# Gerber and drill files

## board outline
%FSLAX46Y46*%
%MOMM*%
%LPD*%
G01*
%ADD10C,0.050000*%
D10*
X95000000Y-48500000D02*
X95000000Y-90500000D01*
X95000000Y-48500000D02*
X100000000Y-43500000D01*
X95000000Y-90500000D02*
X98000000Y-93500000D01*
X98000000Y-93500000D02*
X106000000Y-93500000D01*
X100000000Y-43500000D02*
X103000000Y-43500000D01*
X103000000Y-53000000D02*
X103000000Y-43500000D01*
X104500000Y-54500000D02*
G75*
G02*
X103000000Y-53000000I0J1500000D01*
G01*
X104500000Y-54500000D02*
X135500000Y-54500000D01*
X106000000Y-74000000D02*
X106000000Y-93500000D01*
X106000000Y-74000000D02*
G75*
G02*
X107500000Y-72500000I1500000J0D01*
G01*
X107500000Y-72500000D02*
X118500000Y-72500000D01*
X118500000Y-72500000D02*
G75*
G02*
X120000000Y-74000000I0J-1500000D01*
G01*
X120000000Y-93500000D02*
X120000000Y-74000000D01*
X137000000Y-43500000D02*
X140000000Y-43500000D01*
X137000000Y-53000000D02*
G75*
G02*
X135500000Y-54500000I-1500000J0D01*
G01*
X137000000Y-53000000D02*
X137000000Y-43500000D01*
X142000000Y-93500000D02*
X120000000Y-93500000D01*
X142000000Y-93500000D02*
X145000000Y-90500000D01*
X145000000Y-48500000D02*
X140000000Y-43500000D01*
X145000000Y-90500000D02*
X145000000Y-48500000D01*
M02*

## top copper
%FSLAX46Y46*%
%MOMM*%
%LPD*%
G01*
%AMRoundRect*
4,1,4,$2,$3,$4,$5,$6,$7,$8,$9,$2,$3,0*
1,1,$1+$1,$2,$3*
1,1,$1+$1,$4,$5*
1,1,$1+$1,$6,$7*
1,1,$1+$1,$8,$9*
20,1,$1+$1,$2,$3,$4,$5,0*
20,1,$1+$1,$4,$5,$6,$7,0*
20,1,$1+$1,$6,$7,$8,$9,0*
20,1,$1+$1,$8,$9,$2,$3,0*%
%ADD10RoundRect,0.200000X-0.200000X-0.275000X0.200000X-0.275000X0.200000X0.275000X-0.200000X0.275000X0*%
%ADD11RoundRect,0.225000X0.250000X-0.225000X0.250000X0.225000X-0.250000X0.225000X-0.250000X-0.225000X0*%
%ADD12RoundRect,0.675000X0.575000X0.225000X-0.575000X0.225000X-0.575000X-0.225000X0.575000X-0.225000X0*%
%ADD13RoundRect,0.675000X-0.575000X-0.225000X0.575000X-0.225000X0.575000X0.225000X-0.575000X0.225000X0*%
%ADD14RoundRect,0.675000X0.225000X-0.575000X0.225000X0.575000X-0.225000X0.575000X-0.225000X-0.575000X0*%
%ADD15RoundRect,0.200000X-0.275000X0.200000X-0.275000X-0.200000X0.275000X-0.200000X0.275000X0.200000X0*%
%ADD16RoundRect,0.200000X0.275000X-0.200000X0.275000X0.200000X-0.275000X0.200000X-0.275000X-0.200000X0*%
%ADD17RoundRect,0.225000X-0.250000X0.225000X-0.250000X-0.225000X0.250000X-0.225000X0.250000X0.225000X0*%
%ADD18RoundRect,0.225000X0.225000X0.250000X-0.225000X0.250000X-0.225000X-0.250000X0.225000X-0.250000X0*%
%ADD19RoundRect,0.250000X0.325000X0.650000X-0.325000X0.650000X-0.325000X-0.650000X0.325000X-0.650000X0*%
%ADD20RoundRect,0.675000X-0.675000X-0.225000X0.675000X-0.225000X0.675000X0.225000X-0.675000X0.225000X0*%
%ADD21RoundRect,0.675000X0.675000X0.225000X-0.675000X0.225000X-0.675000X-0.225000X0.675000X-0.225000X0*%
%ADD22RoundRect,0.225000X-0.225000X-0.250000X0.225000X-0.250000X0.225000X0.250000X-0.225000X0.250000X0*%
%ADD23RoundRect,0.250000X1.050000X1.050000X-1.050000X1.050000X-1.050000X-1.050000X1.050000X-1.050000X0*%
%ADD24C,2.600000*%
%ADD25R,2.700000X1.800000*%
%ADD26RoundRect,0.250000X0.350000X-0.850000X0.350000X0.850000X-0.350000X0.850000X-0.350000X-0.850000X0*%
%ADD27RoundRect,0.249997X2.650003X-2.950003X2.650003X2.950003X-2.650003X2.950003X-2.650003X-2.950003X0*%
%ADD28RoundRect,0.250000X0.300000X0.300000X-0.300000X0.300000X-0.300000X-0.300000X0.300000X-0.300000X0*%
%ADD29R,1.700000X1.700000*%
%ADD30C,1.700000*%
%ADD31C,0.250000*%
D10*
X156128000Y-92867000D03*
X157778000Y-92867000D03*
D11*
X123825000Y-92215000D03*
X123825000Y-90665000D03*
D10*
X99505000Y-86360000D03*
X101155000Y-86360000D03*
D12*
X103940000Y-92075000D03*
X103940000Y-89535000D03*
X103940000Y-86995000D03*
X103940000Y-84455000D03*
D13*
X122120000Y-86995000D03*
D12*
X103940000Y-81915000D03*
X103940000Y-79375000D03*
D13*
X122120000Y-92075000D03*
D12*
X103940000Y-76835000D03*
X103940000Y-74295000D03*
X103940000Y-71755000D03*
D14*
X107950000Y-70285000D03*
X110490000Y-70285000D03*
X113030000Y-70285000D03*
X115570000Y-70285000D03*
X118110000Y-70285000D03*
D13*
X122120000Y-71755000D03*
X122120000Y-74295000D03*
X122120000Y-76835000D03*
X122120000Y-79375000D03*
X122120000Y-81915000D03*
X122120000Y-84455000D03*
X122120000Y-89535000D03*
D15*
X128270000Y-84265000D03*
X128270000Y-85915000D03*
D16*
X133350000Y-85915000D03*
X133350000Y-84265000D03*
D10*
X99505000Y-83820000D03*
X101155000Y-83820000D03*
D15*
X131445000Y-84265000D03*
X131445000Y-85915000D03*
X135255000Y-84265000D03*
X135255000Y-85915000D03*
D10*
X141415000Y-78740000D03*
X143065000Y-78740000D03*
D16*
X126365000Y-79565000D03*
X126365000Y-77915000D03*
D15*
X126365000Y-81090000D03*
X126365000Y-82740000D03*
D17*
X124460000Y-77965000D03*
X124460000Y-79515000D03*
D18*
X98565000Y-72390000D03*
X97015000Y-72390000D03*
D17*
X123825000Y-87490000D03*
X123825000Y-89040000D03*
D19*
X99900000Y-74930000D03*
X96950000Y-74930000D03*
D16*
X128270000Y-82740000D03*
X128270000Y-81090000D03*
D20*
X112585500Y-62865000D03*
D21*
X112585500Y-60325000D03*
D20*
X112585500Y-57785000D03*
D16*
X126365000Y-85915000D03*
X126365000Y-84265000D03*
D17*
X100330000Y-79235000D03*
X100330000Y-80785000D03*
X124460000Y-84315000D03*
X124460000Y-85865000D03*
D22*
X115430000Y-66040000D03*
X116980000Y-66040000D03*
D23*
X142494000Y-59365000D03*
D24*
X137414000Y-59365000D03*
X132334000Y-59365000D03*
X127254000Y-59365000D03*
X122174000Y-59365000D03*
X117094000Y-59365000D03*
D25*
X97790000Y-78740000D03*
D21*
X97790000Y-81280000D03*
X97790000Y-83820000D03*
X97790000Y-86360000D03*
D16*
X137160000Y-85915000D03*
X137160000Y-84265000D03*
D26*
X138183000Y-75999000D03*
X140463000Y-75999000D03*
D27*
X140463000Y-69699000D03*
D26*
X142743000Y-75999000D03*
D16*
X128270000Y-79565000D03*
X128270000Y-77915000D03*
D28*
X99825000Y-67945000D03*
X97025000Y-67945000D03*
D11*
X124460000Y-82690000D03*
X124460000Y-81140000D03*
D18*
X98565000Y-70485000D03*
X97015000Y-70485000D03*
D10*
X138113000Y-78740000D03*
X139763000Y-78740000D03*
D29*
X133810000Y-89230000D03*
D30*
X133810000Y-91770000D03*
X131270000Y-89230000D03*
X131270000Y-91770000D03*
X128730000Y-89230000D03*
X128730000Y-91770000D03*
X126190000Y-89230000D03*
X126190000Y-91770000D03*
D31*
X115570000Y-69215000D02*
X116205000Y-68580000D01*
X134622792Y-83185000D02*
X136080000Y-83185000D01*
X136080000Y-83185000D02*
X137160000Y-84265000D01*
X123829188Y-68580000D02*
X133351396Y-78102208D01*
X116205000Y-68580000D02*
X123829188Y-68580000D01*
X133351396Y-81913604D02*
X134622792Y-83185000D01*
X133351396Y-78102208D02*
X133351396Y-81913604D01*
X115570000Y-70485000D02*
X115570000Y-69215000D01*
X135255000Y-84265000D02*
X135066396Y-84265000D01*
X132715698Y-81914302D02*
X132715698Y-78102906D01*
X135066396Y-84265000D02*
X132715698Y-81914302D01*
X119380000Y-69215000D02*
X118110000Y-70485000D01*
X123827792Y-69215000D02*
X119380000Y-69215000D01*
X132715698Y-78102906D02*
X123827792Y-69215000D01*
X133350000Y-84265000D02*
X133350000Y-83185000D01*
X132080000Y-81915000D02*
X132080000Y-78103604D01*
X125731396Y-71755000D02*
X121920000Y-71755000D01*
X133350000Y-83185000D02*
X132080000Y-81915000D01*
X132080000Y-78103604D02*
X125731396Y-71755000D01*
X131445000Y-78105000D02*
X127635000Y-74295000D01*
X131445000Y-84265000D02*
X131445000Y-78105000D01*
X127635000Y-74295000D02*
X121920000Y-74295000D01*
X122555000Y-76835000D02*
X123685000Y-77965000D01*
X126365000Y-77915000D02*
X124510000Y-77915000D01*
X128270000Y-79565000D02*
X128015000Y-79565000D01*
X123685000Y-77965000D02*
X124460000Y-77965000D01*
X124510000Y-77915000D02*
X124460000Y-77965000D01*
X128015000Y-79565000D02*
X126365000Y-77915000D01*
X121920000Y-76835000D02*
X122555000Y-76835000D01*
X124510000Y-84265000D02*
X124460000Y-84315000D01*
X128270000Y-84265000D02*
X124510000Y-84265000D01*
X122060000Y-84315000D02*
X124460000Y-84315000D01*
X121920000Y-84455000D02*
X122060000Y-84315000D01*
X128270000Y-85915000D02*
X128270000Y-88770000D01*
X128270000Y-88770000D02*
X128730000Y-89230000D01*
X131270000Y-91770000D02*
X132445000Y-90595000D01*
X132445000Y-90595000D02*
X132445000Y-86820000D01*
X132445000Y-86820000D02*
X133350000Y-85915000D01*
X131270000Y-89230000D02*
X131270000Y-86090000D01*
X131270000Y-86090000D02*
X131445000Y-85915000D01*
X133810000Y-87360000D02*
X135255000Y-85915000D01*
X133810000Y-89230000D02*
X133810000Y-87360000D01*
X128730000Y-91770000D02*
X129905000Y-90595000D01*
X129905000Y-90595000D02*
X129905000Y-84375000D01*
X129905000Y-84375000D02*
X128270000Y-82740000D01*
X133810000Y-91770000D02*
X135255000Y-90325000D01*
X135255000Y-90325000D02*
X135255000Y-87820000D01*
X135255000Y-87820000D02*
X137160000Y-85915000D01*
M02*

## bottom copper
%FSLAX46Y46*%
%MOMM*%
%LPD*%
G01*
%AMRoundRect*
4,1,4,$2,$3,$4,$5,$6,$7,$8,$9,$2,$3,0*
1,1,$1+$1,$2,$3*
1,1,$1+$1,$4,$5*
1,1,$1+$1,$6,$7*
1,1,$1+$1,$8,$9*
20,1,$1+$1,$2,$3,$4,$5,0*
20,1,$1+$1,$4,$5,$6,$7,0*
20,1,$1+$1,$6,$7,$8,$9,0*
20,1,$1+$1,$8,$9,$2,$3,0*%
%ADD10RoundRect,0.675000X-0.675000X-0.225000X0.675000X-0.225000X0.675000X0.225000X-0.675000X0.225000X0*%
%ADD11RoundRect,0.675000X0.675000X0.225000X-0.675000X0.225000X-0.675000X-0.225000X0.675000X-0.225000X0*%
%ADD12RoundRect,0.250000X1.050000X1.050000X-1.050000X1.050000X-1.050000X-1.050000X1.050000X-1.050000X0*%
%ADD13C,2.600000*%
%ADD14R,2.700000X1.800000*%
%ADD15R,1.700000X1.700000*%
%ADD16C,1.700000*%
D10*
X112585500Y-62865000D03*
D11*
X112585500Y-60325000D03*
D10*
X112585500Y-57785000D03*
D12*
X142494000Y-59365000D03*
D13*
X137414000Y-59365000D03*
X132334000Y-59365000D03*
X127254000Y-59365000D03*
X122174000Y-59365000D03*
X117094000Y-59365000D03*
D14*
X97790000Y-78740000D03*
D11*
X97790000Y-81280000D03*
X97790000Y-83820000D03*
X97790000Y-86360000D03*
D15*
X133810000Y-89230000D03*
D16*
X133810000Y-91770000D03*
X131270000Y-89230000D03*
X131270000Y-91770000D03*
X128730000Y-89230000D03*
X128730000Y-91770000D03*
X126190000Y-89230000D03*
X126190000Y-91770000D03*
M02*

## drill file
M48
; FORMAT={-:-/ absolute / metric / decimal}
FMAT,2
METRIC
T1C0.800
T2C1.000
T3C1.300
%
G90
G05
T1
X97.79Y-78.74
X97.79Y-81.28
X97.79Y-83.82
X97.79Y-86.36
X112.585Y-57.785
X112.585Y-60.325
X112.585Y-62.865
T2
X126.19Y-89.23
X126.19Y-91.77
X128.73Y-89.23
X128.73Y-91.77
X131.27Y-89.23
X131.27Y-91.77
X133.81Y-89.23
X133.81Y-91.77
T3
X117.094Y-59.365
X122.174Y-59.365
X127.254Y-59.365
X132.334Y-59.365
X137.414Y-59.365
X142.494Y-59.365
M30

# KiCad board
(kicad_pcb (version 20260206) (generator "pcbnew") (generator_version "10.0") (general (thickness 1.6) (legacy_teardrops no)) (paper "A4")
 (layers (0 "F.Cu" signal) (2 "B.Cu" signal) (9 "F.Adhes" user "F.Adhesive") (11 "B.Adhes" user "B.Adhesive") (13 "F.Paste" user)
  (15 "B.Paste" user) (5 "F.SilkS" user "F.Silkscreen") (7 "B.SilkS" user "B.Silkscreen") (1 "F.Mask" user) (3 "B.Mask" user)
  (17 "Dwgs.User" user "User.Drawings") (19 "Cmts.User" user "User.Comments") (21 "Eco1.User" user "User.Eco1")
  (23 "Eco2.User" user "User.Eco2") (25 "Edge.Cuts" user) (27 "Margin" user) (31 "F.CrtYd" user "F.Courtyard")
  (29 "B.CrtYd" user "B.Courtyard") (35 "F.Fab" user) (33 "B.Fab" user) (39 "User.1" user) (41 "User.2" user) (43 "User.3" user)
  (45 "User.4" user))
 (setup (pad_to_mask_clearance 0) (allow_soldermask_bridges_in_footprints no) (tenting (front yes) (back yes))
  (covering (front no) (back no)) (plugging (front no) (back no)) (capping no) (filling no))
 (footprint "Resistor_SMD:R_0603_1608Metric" (layer "F.Cu") (at 156.953 92.867)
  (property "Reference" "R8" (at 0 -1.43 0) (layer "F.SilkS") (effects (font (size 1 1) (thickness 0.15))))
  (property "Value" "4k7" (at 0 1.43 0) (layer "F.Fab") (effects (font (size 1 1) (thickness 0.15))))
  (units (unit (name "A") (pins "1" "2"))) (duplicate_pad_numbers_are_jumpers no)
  (pad "1" smd roundrect (at -0.825 0) (size 0.8 0.95) (layers "F.Cu" "F.Mask" "F.Paste") (roundrect_rratio 0.25) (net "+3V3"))
  (pad "2" smd roundrect (at 0.825 0) (size 0.8 0.95) (layers "F.Cu" "F.Mask" "F.Paste") (roundrect_rratio 0.25) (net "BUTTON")))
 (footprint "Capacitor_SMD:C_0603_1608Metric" (layer "F.Cu") (at 123.825 91.44 90)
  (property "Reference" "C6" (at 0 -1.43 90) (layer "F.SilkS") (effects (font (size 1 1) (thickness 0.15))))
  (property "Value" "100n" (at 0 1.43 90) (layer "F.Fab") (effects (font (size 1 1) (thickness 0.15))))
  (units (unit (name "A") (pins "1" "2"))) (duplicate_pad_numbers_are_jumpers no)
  (pad "1" smd roundrect (at -0.775 0 90) (size 0.9 0.95) (layers "F.Cu" "F.Mask" "F.Paste") (roundrect_rratio 0.25) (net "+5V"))
  (pad "2" smd roundrect (at 0.775 0 90) (size 0.9 0.95) (layers "F.Cu" "F.Mask" "F.Paste") (roundrect_rratio 0.25) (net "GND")))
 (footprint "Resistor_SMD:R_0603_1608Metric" (layer "F.Cu") (at 100.33 86.36)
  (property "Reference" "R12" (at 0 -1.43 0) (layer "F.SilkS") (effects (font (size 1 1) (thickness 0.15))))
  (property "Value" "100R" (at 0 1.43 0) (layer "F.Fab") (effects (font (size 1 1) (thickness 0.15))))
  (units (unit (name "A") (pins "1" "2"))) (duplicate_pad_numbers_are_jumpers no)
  (pad "1" smd roundrect (at -0.825 0) (size 0.8 0.95) (layers "F.Cu" "F.Mask" "F.Paste") (roundrect_rratio 0.25) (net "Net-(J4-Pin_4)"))
  (pad "2" smd roundrect (at 0.825 0) (size 0.8 0.95) (layers "F.Cu" "F.Mask" "F.Paste") (roundrect_rratio 0.25) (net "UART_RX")))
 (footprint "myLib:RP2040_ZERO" (layer "F.Cu") (at 113.03 80.645 180)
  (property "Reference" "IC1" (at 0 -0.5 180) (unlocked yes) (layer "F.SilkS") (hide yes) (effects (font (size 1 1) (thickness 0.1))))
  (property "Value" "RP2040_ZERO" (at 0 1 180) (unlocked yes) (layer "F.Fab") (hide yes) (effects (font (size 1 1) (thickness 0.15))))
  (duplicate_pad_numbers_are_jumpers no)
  (pad "0" smd roundrect (at 8.89 -11.43 180) (size 2.5 1.8) (drill (offset 0.2 0)) (layers "F.Cu" "F.Mask" "F.Paste")
   (roundrect_rratio 0.375) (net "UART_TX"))
  (pad "1" smd roundrect (at 8.89 -8.89 180) (size 2.5 1.8) (drill (offset 0.2 0)) (layers "F.Cu" "F.Mask" "F.Paste")
   (roundrect_rratio 0.375) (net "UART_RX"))
  (pad "2" smd roundrect (at 8.89 -6.35 180) (size 2.5 1.8) (drill (offset 0.2 0)) (layers "F.Cu" "F.Mask" "F.Paste")
   (roundrect_rratio 0.375) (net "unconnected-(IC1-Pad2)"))
  (pad "3" smd roundrect (at 8.89 -3.81 180) (size 2.5 1.8) (drill (offset 0.2 0)) (layers "F.Cu" "F.Mask" "F.Paste")
   (roundrect_rratio 0.375) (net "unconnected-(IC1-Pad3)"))
  (pad "3V3" smd roundrect (at -8.89 -6.35) (size 2.5 1.8) (drill (offset 0.2 0)) (layers "F.Cu" "F.Mask" "F.Paste")
   (roundrect_rratio 0.375) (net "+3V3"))
  (pad "4" smd roundrect (at 8.89 -1.27 180) (size 2.5 1.8) (drill (offset 0.2 0)) (layers "F.Cu" "F.Mask" "F.Paste")
   (roundrect_rratio 0.375) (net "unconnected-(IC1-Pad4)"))
  (pad "5" smd roundrect (at 8.89 1.27 180) (size 2.5 1.8) (drill (offset 0.2 0)) (layers "F.Cu" "F.Mask" "F.Paste")
   (roundrect_rratio 0.375) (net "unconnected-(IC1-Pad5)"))
  (pad "5V0" smd roundrect (at -8.89 -11.43) (size 2.5 1.8) (drill (offset 0.2 0)) (layers "F.Cu" "F.Mask" "F.Paste")
   (roundrect_rratio 0.375) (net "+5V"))
  (pad "6" smd roundrect (at 8.89 3.81 180) (size 2.5 1.8) (drill (offset 0.2 0)) (layers "F.Cu" "F.Mask" "F.Paste")
   (roundrect_rratio 0.375) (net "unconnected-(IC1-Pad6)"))
  (pad "7" smd roundrect (at 8.89 6.35 180) (size 2.5 1.8) (drill (offset 0.2 0)) (layers "F.Cu" "F.Mask" "F.Paste")
   (roundrect_rratio 0.375) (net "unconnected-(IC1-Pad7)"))
  (pad "8" smd roundrect (at 8.89 8.89 180) (size 2.5 1.8) (drill (offset 0.2 0)) (layers "F.Cu" "F.Mask" "F.Paste")
   (roundrect_rratio 0.375) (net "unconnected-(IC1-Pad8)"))
  (pad "9" smd roundrect (at 5.08 10.16 90) (size 2.5 1.8) (drill (offset 0.2 0)) (layers "F.Cu" "F.Mask" "F.Paste")
   (roundrect_rratio 0.375) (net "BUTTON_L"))
  (pad "10" smd roundrect (at 2.54 10.16 90) (size 2.5 1.8) (drill (offset 0.2 0)) (layers "F.Cu" "F.Mask" "F.Paste")
   (roundrect_rratio 0.375) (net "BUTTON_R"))
  (pad "11" smd roundrect (at 0 10.16 90) (size 2.5 1.8) (drill (offset 0.2 0)) (layers "F.Cu" "F.Mask" "F.Paste") (roundrect_rratio 0.375)
   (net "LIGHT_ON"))
  (pad "12" smd roundrect (at -2.54 10.16 90) (size 2.5 1.8) (drill (offset 0.2 0)) (layers "F.Cu" "F.Mask" "F.Paste")
   (roundrect_rratio 0.375) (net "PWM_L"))
  (pad "13" smd roundrect (at -5.08 10.16 90) (size 2.5 1.8) (drill (offset 0.2 0)) (layers "F.Cu" "F.Mask" "F.Paste")
   (roundrect_rratio 0.375) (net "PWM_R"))
  (pad "14" smd roundrect (at -8.89 8.89) (size 2.5 1.8) (drill (offset 0.2 0)) (layers "F.Cu" "F.Mask" "F.Paste") (roundrect_rratio 0.375)
   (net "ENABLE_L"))
  (pad "15" smd roundrect (at -8.89 6.35) (size 2.5 1.8) (drill (offset 0.2 0)) (layers "F.Cu" "F.Mask" "F.Paste") (roundrect_rratio 0.375)
   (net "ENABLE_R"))
  (pad "26" smd roundrect (at -8.89 3.81) (size 2.5 1.8) (drill (offset 0.2 0)) (layers "F.Cu" "F.Mask" "F.Paste") (roundrect_rratio 0.375)
   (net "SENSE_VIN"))
  (pad "27" smd roundrect (at -8.89 1.27) (size 2.5 1.8) (drill (offset 0.2 0)) (layers "F.Cu" "F.Mask" "F.Paste") (roundrect_rratio 0.375)
   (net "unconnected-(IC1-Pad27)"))
  (pad "28" smd roundrect (at -8.89 -1.27) (size 2.5 1.8) (drill (offset 0.2 0)) (layers "F.Cu" "F.Mask" "F.Paste") (roundrect_rratio 0.375)
   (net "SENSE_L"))
  (pad "29" smd roundrect (at -8.89 -3.81) (size 2.5 1.8) (drill (offset 0.2 0)) (layers "F.Cu" "F.Mask" "F.Paste") (roundrect_rratio 0.375)
   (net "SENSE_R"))
  (pad "GND" smd roundrect (at -8.89 -8.89) (size 2.5 1.8) (drill (offset 0.2 0)) (layers "F.Cu" "F.Mask" "F.Paste")
   (roundrect_rratio 0.375) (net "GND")))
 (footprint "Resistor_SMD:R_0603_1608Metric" (layer "F.Cu") (at 128.27 85.09 -90)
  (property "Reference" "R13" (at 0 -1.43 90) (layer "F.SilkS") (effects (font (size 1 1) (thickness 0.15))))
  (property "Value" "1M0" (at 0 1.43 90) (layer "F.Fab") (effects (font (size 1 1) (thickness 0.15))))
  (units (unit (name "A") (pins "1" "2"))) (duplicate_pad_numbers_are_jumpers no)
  (pad "1" smd roundrect (at -0.825 0 270) (size 0.8 0.95) (layers "F.Cu" "F.Mask" "F.Paste") (roundrect_rratio 0.25) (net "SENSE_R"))
  (pad "2" smd roundrect (at 0.825 0 270) (size 0.8 0.95) (layers "F.Cu" "F.Mask" "F.Paste") (roundrect_rratio 0.25) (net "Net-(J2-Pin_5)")))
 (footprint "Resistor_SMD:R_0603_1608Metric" (layer "F.Cu") (at 133.35 85.09 90)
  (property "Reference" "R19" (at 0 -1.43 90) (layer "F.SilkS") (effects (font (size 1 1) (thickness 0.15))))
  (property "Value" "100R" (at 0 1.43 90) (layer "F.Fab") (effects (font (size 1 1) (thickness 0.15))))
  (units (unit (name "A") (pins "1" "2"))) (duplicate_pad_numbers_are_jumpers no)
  (pad "1" smd roundrect (at -0.825 0 90) (size 0.8 0.95) (layers "F.Cu" "F.Mask" "F.Paste") (roundrect_rratio 0.25) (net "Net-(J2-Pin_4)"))
  (pad "2" smd roundrect (at 0.825 0 90) (size 0.8 0.95) (layers "F.Cu" "F.Mask" "F.Paste") (roundrect_rratio 0.25) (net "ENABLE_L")))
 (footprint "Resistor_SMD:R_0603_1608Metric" (layer "F.Cu") (at 100.33 83.82)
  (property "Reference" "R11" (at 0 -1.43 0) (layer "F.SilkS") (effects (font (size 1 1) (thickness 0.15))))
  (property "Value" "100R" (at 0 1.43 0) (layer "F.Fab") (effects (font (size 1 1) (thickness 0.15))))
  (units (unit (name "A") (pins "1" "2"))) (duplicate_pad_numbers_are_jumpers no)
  (pad "1" smd roundrect (at -0.825 0) (size 0.8 0.95) (layers "F.Cu" "F.Mask" "F.Paste") (roundrect_rratio 0.25) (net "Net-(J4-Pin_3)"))
  (pad "2" smd roundrect (at 0.825 0) (size 0.8 0.95) (layers "F.Cu" "F.Mask" "F.Paste") (roundrect_rratio 0.25) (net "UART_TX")))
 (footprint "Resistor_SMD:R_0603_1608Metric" (layer "F.Cu") (at 131.445 85.09 -90)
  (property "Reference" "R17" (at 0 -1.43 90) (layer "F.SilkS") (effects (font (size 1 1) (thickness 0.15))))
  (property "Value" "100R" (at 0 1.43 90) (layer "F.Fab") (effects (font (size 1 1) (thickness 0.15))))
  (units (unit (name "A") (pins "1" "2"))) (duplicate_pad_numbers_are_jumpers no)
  (pad "1" smd roundrect (at -0.825 0 270) (size 0.8 0.95) (layers "F.Cu" "F.Mask" "F.Paste") (roundrect_rratio 0.25) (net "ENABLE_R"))
  (pad "2" smd roundrect (at 0.825 0 270) (size 0.8 0.95) (layers "F.Cu" "F.Mask" "F.Paste") (roundrect_rratio 0.25) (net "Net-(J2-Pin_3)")))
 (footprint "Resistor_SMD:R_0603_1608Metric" (layer "F.Cu") (at 135.255 85.09 -90)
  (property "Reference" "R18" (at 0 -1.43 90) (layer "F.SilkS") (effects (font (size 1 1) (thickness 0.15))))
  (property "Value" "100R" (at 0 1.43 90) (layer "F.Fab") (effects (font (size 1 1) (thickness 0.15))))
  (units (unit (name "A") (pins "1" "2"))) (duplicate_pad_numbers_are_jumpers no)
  (pad "1" smd roundrect (at -0.825 0 270) (size 0.8 0.95) (layers "F.Cu" "F.Mask" "F.Paste") (roundrect_rratio 0.25) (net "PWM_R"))
  (pad "2" smd roundrect (at 0.825 0 270) (size 0.8 0.95) (layers "F.Cu" "F.Mask" "F.Paste") (roundrect_rratio 0.25) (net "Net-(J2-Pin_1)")))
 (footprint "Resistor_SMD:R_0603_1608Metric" (layer "F.Cu") (at 142.24 78.74)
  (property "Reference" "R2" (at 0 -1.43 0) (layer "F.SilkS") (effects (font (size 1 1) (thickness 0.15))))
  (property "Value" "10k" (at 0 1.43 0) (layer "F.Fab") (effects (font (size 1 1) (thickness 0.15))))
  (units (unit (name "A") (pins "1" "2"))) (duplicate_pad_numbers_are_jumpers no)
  (pad "1" smd roundrect (at -0.825 0) (size 0.8 0.95) (layers "F.Cu" "F.Mask" "F.Paste") (roundrect_rratio 0.25) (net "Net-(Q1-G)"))
  (pad "2" smd roundrect (at 0.825 0) (size 0.8 0.95) (layers "F.Cu" "F.Mask" "F.Paste") (roundrect_rratio 0.25) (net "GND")))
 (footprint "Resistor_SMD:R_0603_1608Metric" (layer "F.Cu") (at 126.365 78.74 90)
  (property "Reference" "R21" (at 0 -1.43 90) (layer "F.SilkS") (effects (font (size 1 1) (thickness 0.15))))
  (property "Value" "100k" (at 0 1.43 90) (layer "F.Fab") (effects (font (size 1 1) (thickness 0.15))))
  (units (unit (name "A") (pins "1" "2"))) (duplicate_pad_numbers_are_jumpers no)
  (pad "1" smd roundrect (at -0.825 0 90) (size 0.8 0.95) (layers "F.Cu" "F.Mask" "F.Paste") (roundrect_rratio 0.25) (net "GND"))
  (pad "2" smd roundrect (at 0.825 0 90) (size 0.8 0.95) (layers "F.Cu" "F.Mask" "F.Paste") (roundrect_rratio 0.25) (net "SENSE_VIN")))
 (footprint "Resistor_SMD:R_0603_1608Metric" (layer "F.Cu") (at 126.365 81.915 -90)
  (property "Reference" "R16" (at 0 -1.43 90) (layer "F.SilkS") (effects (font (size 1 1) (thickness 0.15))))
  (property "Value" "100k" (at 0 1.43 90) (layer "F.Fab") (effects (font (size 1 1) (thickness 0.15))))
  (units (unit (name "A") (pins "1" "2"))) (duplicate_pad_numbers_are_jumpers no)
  (pad "1" smd roundrect (at -0.825 0 270) (size 0.8 0.95) (layers "F.Cu" "F.Mask" "F.Paste") (roundrect_rratio 0.25) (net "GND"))
  (pad "2" smd roundrect (at 0.825 0 270) (size 0.8 0.95) (layers "F.Cu" "F.Mask" "F.Paste") (roundrect_rratio 0.25) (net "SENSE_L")))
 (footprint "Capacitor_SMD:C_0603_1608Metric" (layer "F.Cu") (at 124.46 78.74 -90)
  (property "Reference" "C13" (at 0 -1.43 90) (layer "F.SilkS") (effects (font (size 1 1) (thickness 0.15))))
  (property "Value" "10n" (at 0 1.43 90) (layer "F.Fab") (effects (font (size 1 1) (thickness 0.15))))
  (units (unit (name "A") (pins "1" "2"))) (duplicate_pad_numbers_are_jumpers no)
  (pad "1" smd roundrect (at -0.775 0 270) (size 0.9 0.95) (layers "F.Cu" "F.Mask" "F.Paste") (roundrect_rratio 0.25) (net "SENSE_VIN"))
  (pad "2" smd roundrect (at 0.775 0 270) (size 0.9 0.95) (layers "F.Cu" "F.Mask" "F.Paste") (roundrect_rratio 0.25) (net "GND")))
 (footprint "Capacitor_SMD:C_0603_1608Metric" (layer "F.Cu") (at 97.79 72.39 180)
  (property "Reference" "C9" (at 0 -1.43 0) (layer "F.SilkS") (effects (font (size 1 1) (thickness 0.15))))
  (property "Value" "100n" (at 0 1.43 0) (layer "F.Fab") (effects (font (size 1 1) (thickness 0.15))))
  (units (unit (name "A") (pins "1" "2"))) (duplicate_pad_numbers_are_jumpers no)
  (pad "1" smd roundrect (at -0.775 0 180) (size 0.9 0.95) (layers "F.Cu" "F.Mask" "F.Paste") (roundrect_rratio 0.25) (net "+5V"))
  (pad "2" smd roundrect (at 0.775 0 180) (size 0.9 0.95) (layers "F.Cu" "F.Mask" "F.Paste") (roundrect_rratio 0.25) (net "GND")))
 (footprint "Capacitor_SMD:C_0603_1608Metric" (layer "F.Cu") (at 123.825 88.265 -90)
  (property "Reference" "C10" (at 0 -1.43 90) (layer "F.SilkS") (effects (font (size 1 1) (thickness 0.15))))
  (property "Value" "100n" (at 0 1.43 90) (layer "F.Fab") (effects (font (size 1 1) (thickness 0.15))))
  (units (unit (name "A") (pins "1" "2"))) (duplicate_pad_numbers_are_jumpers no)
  (pad "1" smd roundrect (at -0.775 0 270) (size 0.9 0.95) (layers "F.Cu" "F.Mask" "F.Paste") (roundrect_rratio 0.25) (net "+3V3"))
  (pad "2" smd roundrect (at 0.775 0 270) (size 0.9 0.95) (layers "F.Cu" "F.Mask" "F.Paste") (roundrect_rratio 0.25) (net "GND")))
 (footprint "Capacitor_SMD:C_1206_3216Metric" (layer "F.Cu") (at 98.425 74.93 180)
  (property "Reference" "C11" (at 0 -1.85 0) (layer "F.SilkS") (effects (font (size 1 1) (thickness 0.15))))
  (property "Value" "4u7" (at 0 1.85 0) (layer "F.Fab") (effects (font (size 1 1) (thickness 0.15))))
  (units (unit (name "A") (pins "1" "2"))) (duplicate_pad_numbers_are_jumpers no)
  (pad "1" smd roundrect (at -1.475 0 180) (size 1.15 1.8) (layers "F.Cu" "F.Mask" "F.Paste") (roundrect_rratio 0.217391) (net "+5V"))
  (pad "2" smd roundrect (at 1.475 0 180) (size 1.15 1.8) (layers "F.Cu" "F.Mask" "F.Paste") (roundrect_rratio 0.217391) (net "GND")))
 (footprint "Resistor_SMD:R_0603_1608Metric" (layer "F.Cu") (at 128.27 81.915 90)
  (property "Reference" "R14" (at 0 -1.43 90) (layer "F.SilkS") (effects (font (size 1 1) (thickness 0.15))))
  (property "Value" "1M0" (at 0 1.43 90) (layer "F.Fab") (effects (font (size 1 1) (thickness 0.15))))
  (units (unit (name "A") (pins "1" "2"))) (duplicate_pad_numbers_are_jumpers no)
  (pad "1" smd roundrect (at -0.825 0 90) (size 0.8 0.95) (layers "F.Cu" "F.Mask" "F.Paste") (roundrect_rratio 0.25) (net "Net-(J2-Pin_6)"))
  (pad "2" smd roundrect (at 0.825 0 90) (size 0.8 0.95) (layers "F.Cu" "F.Mask" "F.Paste") (roundrect_rratio 0.25) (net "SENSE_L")))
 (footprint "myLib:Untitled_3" (layer "F.Cu") (at 107.5055 60.325 90)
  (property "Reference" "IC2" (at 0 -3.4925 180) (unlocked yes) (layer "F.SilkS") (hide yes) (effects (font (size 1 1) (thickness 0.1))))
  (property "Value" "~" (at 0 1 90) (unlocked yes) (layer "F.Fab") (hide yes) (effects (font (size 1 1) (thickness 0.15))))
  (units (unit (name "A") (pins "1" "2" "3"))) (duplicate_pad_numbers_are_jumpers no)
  (pad "1" thru_hole roundrect (at -2.54 5.08) (size 2.7 1.8) (drill 0.8) (layers "*.Cu" "*.Mask") (remove_unused_layers no)
   (roundrect_rratio 0.375) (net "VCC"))
  (pad "2" thru_hole roundrect (at 0 5.08 180) (size 2.7 1.8) (drill 0.8) (layers "*.Cu" "*.Mask") (remove_unused_layers no)
   (roundrect_rratio 0.375) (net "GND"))
  (pad "3" thru_hole roundrect (at 2.54 5.08) (size 2.7 1.8) (drill 0.8) (layers "*.Cu" "*.Mask") (remove_unused_layers no)
   (roundrect_rratio 0.375) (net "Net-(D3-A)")))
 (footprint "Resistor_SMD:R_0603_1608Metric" (layer "F.Cu") (at 126.365 85.09 90)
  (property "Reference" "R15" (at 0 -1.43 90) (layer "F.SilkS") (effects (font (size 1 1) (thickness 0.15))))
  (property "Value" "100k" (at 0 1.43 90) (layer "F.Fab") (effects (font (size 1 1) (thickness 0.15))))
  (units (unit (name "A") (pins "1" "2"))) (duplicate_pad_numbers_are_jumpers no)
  (pad "1" smd roundrect (at -0.825 0 90) (size 0.8 0.95) (layers "F.Cu" "F.Mask" "F.Paste") (roundrect_rratio 0.25) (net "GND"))
  (pad "2" smd roundrect (at 0.825 0 90) (size 0.8 0.95) (layers "F.Cu" "F.Mask" "F.Paste") (roundrect_rratio 0.25) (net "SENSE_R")))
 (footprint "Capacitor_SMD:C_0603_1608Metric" (layer "F.Cu") (at 100.33 80.01 -90)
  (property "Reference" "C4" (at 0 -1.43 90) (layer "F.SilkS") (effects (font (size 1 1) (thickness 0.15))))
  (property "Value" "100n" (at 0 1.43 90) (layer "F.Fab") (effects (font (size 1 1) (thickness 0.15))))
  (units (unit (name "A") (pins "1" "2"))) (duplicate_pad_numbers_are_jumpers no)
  (pad "1" smd roundrect (at -0.775 0 270) (size 0.9 0.95) (layers "F.Cu" "F.Mask" "F.Paste") (roundrect_rratio 0.25) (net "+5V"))
  (pad "2" smd roundrect (at 0.775 0 270) (size 0.9 0.95) (layers "F.Cu" "F.Mask" "F.Paste") (roundrect_rratio 0.25) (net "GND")))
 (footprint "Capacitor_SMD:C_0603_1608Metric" (layer "F.Cu") (at 124.46 85.09 -90)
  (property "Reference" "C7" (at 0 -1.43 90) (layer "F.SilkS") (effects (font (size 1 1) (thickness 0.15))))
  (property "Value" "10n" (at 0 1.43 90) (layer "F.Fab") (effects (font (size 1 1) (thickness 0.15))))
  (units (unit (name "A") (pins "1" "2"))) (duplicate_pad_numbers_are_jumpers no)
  (pad "1" smd roundrect (at -0.775 0 270) (size 0.9 0.95) (layers "F.Cu" "F.Mask" "F.Paste") (roundrect_rratio 0.25) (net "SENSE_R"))
  (pad "2" smd roundrect (at 0.775 0 270) (size 0.9 0.95) (layers "F.Cu" "F.Mask" "F.Paste") (roundrect_rratio 0.25) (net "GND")))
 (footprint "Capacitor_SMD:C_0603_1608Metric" (layer "F.Cu") (at 116.205 66.04)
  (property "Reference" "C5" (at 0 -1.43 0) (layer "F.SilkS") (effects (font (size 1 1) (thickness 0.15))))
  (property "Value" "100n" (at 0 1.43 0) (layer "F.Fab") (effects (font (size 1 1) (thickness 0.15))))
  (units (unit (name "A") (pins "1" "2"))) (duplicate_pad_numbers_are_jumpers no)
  (pad "1" smd roundrect (at -0.775 0) (size 0.9 0.95) (layers "F.Cu" "F.Mask" "F.Paste") (roundrect_rratio 0.25) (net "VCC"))
  (pad "2" smd roundrect (at 0.775 0) (size 0.9 0.95) (layers "F.Cu" "F.Mask" "F.Paste") (roundrect_rratio 0.25) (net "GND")))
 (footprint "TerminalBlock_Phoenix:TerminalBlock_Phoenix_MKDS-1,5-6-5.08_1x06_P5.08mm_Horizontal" (layer "F.Cu") (at 142.494 59.365 180)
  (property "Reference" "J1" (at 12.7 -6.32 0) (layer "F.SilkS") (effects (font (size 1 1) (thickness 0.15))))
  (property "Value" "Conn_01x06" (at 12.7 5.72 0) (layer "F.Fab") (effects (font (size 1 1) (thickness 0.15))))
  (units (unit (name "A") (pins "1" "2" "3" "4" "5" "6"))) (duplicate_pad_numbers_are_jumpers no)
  (pad "1" thru_hole roundrect (at 0 0 180) (size 2.6 2.6) (drill 1.3) (layers "*.Cu" "*.Mask") (remove_unused_layers no)
   (roundrect_rratio 0.096154) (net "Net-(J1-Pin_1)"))
  (pad "2" thru_hole circle (at 5.08 0 180) (size 2.6 2.6) (drill 1.3) (layers "*.Cu" "*.Mask") (remove_unused_layers no)
   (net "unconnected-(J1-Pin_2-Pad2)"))
  (pad "3" thru_hole circle (at 10.16 0 180) (size 2.6 2.6) (drill 1.3) (layers "*.Cu" "*.Mask") (remove_unused_layers no)
   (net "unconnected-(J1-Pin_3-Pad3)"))
  (pad "4" thru_hole circle (at 15.24 0 180) (size 2.6 2.6) (drill 1.3) (layers "*.Cu" "*.Mask") (remove_unused_layers no)
   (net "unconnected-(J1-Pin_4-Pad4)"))
  (pad "5" thru_hole circle (at 20.32 0 180) (size 2.6 2.6) (drill 1.3) (layers "*.Cu" "*.Mask") (remove_unused_layers no) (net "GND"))
  (pad "6" thru_hole circle (at 25.4 0 180) (size 2.6 2.6) (drill 1.3) (layers "*.Cu" "*.Mask") (remove_unused_layers no) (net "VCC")))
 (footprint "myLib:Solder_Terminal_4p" (layer "F.Cu") (at 97.79 82.55 -90)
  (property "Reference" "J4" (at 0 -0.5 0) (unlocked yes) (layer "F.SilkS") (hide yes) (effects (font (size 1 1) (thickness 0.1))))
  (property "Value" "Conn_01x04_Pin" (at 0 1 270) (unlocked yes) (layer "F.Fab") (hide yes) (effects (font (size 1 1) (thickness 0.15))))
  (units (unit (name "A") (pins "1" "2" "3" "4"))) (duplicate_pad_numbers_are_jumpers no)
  (pad "1" thru_hole rect (at -3.81 0 180) (size 2.7 1.8) (drill 0.8) (layers "*.Cu" "*.Mask") (remove_unused_layers no) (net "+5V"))
  (pad "2" thru_hole roundrect (at -1.27 0 180) (size 2.7 1.8) (drill 0.8) (layers "*.Cu" "*.Mask") (remove_unused_layers no)
   (roundrect_rratio 0.375) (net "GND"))
  (pad "3" thru_hole roundrect (at 1.27 0 180) (size 2.7 1.8) (drill 0.8) (layers "*.Cu" "*.Mask") (remove_unused_layers no)
   (roundrect_rratio 0.375) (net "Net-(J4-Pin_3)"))
  (pad "4" thru_hole roundrect (at 3.81 0 180) (size 2.7 1.8) (drill 0.8) (layers "*.Cu" "*.Mask") (remove_unused_layers no)
   (roundrect_rratio 0.375) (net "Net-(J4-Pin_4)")))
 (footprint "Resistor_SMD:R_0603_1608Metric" (layer "F.Cu") (at 137.16 85.09 90)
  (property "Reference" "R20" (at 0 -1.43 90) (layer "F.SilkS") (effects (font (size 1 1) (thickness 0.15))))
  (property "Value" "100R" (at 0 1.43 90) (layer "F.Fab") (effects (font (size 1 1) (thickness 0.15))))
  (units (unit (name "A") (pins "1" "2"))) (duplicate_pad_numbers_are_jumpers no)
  (pad "1" smd roundrect (at -0.825 0 90) (size 0.8 0.95) (layers "F.Cu" "F.Mask" "F.Paste") (roundrect_rratio 0.25) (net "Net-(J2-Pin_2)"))
  (pad "2" smd roundrect (at 0.825 0 90) (size 0.8 0.95) (layers "F.Cu" "F.Mask" "F.Paste") (roundrect_rratio 0.25) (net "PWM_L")))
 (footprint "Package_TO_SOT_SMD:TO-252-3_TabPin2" (layer "F.Cu") (at 140.463 70.959 90)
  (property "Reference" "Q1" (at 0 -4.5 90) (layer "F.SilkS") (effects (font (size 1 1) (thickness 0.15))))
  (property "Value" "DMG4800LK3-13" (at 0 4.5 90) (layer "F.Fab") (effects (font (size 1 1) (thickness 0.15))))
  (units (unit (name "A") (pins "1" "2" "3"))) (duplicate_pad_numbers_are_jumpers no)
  (pad "" smd roundrect (at -0.415 -1.525 90) (size 3.05 2.75) (layers "F.Paste") (roundrect_rratio 0.090909))
  (pad "" smd roundrect (at -0.415 1.525 90) (size 3.05 2.75) (layers "F.Paste") (roundrect_rratio 0.090909))
  (pad "" smd roundrect (at 2.935 -1.525 90) (size 3.05 2.75) (layers "F.Paste") (roundrect_rratio 0.090909))
  (pad "" smd roundrect (at 2.935 1.525 90) (size 3.05 2.75) (layers "F.Paste") (roundrect_rratio 0.090909))
  (pad "1" smd roundrect (at -5.04 -2.28 90) (size 2.2 1.2) (layers "F.Cu" "F.Mask" "F.Paste") (roundrect_rratio 0.208333)
   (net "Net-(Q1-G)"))
  (pad "2" smd roundrect (at -5.04 0 90) (size 2.2 1.2) (layers "F.Cu" "F.Mask" "F.Paste") (roundrect_rratio 0.208333)
   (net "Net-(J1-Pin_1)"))
  (pad "2" smd roundrect (at 1.26 0 90) (size 6.4 5.8) (layers "F.Cu" "F.Mask") (roundrect_rratio 0.043103) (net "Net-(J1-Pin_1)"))
  (pad "3" smd roundrect (at -5.04 2.28 90) (size 2.2 1.2) (layers "F.Cu" "F.Mask" "F.Paste") (roundrect_rratio 0.208333) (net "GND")))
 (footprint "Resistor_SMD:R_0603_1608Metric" (layer "F.Cu") (at 128.27 78.74 90)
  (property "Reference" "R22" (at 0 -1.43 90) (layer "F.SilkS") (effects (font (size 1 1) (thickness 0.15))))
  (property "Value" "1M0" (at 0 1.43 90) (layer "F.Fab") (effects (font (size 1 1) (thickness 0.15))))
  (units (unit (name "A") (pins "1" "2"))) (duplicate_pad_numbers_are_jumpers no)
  (pad "1" smd roundrect (at -0.825 0 90) (size 0.8 0.95) (layers "F.Cu" "F.Mask" "F.Paste") (roundrect_rratio 0.25) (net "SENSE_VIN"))
  (pad "2" smd roundrect (at 0.825 0 90) (size 0.8 0.95) (layers "F.Cu" "F.Mask" "F.Paste") (roundrect_rratio 0.25) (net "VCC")))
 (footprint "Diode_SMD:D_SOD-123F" (layer "F.Cu") (at 98.425 67.945 180)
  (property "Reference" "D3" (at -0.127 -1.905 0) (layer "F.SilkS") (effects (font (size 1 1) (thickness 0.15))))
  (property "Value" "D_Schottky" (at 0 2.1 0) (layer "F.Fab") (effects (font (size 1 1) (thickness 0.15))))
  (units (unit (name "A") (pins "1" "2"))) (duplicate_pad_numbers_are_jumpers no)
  (pad "1" smd roundrect (at -1.4 0 180) (size 1.1 1.1) (layers "F.Cu" "F.Mask" "F.Paste") (roundrect_rratio 0.2272727273) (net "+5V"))
  (pad "2" smd roundrect (at 1.4 0 180) (size 1.1 1.1) (layers "F.Cu" "F.Mask" "F.Paste") (roundrect_rratio 0.2272727273) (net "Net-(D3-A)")))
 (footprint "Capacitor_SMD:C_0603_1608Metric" (layer "F.Cu") (at 124.46 81.915 90)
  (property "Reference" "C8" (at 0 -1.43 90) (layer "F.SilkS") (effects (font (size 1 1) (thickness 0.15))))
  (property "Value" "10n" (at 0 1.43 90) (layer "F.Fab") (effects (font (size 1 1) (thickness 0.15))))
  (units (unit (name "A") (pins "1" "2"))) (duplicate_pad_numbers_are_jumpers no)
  (pad "1" smd roundrect (at -0.775 0 90) (size 0.9 0.95) (layers "F.Cu" "F.Mask" "F.Paste") (roundrect_rratio 0.25) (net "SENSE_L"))
  (pad "2" smd roundrect (at 0.775 0 90) (size 0.9 0.95) (layers "F.Cu" "F.Mask" "F.Paste") (roundrect_rratio 0.25) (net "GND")))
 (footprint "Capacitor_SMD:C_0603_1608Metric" (layer "F.Cu") (at 97.79 70.485 180)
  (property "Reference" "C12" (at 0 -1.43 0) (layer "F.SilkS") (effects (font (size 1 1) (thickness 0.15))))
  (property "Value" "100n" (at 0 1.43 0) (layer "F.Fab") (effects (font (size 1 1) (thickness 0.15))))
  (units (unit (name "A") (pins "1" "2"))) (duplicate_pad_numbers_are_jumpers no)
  (pad "1" smd roundrect (at -0.775 0 180) (size 0.9 0.95) (layers "F.Cu" "F.Mask" "F.Paste") (roundrect_rratio 0.25) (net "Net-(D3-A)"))
  (pad "2" smd roundrect (at 0.775 0 180) (size 0.9 0.95) (layers "F.Cu" "F.Mask" "F.Paste") (roundrect_rratio 0.25) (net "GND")))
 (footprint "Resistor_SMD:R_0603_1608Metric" (layer "F.Cu") (at 138.938 78.74)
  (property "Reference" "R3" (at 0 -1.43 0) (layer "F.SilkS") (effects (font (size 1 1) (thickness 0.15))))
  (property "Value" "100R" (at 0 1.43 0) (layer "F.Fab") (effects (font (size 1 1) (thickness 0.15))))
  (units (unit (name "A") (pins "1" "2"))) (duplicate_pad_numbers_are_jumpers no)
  (pad "1" smd roundrect (at -0.825 0) (size 0.8 0.95) (layers "F.Cu" "F.Mask" "F.Paste") (roundrect_rratio 0.25) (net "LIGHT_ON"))
  (pad "2" smd roundrect (at 0.825 0) (size 0.8 0.95) (layers "F.Cu" "F.Mask" "F.Paste") (roundrect_rratio 0.25) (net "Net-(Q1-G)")))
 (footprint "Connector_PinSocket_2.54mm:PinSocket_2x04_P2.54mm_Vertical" (layer "B.Cu") (at 133.81 89.23 90)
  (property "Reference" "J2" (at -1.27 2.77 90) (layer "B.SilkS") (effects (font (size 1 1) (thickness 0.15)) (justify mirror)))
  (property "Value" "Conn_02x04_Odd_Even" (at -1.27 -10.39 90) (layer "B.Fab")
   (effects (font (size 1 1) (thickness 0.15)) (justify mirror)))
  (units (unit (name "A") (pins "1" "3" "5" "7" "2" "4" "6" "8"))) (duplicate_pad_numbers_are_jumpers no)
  (pad "1" thru_hole rect (at 0 0 90) (size 1.7 1.7) (drill 1) (layers "*.Cu" "*.Mask") (remove_unused_layers no) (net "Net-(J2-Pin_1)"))
  (pad "2" thru_hole circle (at -2.54 0 90) (size 1.7 1.7) (drill 1) (layers "*.Cu" "*.Mask") (remove_unused_layers no)
   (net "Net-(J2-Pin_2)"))
  (pad "3" thru_hole circle (at 0 -2.54 90) (size 1.7 1.7) (drill 1) (layers "*.Cu" "*.Mask") (remove_unused_layers no)
   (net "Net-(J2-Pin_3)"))
  (pad "4" thru_hole circle (at -2.54 -2.54 90) (size 1.7 1.7) (drill 1) (layers "*.Cu" "*.Mask") (remove_unused_layers no)
   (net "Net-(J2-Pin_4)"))
  (pad "5" thru_hole circle (at 0 -5.08 90) (size 1.7 1.7) (drill 1) (layers "*.Cu" "*.Mask") (remove_unused_layers no)
   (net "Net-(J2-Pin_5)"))
  (pad "6" thru_hole circle (at -2.54 -5.08 90) (size 1.7 1.7) (drill 1) (layers "*.Cu" "*.Mask") (remove_unused_layers no)
   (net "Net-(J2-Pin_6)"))
  (pad "7" thru_hole circle (at 0 -7.62 90) (size 1.7 1.7) (drill 1) (layers "*.Cu" "*.Mask") (remove_unused_layers no) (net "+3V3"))
  (pad "8" thru_hole circle (at -2.54 -7.62 90) (size 1.7 1.7) (drill 1) (layers "*.Cu" "*.Mask") (remove_unused_layers no) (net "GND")))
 (gr_line (start 95 48.5) (end 95 90.5) (stroke (width 0.05) (type default)) (layer "Edge.Cuts"))
 (gr_line (start 95 48.5) (end 100 43.5) (stroke (width 0.05) (type default)) (layer "Edge.Cuts"))
 (gr_line (start 95 90.5) (end 98 93.5) (stroke (width 0.05) (type default)) (layer "Edge.Cuts"))
 (gr_line (start 98 93.5) (end 106 93.5) (stroke (width 0.05) (type default)) (layer "Edge.Cuts"))
 (gr_line (start 100 43.5) (end 103 43.5) (stroke (width 0.05) (type default)) (layer "Edge.Cuts"))
 (gr_line (start 103 53) (end 103 43.5) (stroke (width 0.05) (type default)) (layer "Edge.Cuts"))
 (gr_arc (start 104.5 54.5) (mid 103.43934 54.06066) (end 103 53) (stroke (width 0.05) (type default)) (layer "Edge.Cuts"))
 (gr_line (start 104.5 54.5) (end 135.5 54.5) (stroke (width 0.05) (type default)) (layer "Edge.Cuts"))
 (gr_line (start 106 74) (end 106 93.5) (stroke (width 0.05) (type default)) (layer "Edge.Cuts"))
 (gr_arc (start 106 74) (mid 106.43934 72.93934) (end 107.5 72.5) (stroke (width 0.05) (type default)) (layer "Edge.Cuts"))
 (gr_line (start 107.5 72.5) (end 118.5 72.5) (stroke (width 0.05) (type default)) (layer "Edge.Cuts"))
 (gr_arc (start 118.5 72.5) (mid 119.56066 72.93934) (end 120 74) (stroke (width 0.05) (type default)) (layer "Edge.Cuts"))
 (gr_line (start 120 93.5) (end 120 74) (stroke (width 0.05) (type default)) (layer "Edge.Cuts"))
 (gr_line (start 137 43.5) (end 140 43.5) (stroke (width 0.05) (type default)) (layer "Edge.Cuts"))
 (gr_arc (start 137 53) (mid 136.56066 54.06066) (end 135.5 54.5) (stroke (width 0.05) (type default)) (layer "Edge.Cuts"))
 (gr_line (start 137 53) (end 137 43.5) (stroke (width 0.05) (type default)) (layer "Edge.Cuts"))
 (gr_line (start 142 93.5) (end 120 93.5) (stroke (width 0.05) (type default)) (layer "Edge.Cuts"))
 (gr_line (start 142 93.5) (end 145 90.5) (stroke (width 0.05) (type default)) (layer "Edge.Cuts"))
 (gr_line (start 145 48.5) (end 140 43.5) (stroke (width 0.05) (type default)) (layer "Edge.Cuts"))
 (gr_line (start 145 90.5) (end 145 48.5) (stroke (width 0.05) (type default)) (layer "Edge.Cuts"))
 (segment (start 115.57 69.215) (end 116.205 68.58) (width 0.25) (layer "F.Cu") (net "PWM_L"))
 (segment (start 134.622792 83.185) (end 136.08 83.185) (width 0.25) (layer "F.Cu") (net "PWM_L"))
 (segment (start 136.08 83.185) (end 137.16 84.265) (width 0.25) (layer "F.Cu") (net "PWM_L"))
 (segment (start 123.829188 68.58) (end 133.351396 78.102208) (width 0.25) (layer "F.Cu") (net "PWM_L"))
 (segment (start 116.205 68.58) (end 123.829188 68.58) (width 0.25) (layer "F.Cu") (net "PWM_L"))
 (segment (start 133.351396 81.913604) (end 134.622792 83.185) (width 0.25) (layer "F.Cu") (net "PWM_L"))
 (segment (start 133.351396 78.102208) (end 133.351396 81.913604) (width 0.25) (layer "F.Cu") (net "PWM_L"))
 (segment (start 115.57 70.485) (end 115.57 69.215) (width 0.25) (layer "F.Cu") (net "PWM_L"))
 (segment (start 135.255 84.265) (end 135.066396 84.265) (width 0.25) (layer "F.Cu") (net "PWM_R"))
 (segment (start 132.715698 81.914302) (end 132.715698 78.102906) (width 0.25) (layer "F.Cu") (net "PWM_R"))
 (segment (start 135.066396 84.265) (end 132.715698 81.914302) (width 0.25) (layer "F.Cu") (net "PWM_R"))
 (segment (start 119.38 69.215) (end 118.11 70.485) (width 0.25) (layer "F.Cu") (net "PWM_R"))
 (segment (start 123.827792 69.215) (end 119.38 69.215) (width 0.25) (layer "F.Cu") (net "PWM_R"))
 (segment (start 132.715698 78.102906) (end 123.827792 69.215) (width 0.25) (layer "F.Cu") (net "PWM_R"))
 (segment (start 133.35 84.265) (end 133.35 83.185) (width 0.25) (layer "F.Cu") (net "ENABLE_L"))
 (segment (start 132.08 81.915) (end 132.08 78.103604) (width 0.25) (layer "F.Cu") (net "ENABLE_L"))
 (segment (start 125.731396 71.755) (end 121.92 71.755) (width 0.25) (layer "F.Cu") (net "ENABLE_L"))
 (segment (start 133.35 83.185) (end 132.08 81.915) (width 0.25) (layer "F.Cu") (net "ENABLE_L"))
 (segment (start 132.08 78.103604) (end 125.731396 71.755) (width 0.25) (layer "F.Cu") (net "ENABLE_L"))
 (segment (start 131.445 78.105) (end 127.635 74.295) (width 0.25) (layer "F.Cu") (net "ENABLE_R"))
 (segment (start 131.445 84.265) (end 131.445 78.105) (width 0.25) (layer "F.Cu") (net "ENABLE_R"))
 (segment (start 127.635 74.295) (end 121.92 74.295) (width 0.25) (layer "F.Cu") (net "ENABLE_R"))
 (segment (start 122.555 76.835) (end 123.685 77.965) (width 0.25) (layer "F.Cu") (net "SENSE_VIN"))
 (segment (start 126.365 77.915) (end 124.51 77.915) (width 0.25) (layer "F.Cu") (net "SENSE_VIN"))
 (segment (start 128.27 79.565) (end 128.015 79.565) (width 0.25) (layer "F.Cu") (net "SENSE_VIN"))
 (segment (start 123.685 77.965) (end 124.46 77.965) (width 0.25) (layer "F.Cu") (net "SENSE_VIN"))
 (segment (start 124.51 77.915) (end 124.46 77.965) (width 0.25) (layer "F.Cu") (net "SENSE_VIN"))
 (segment (start 128.015 79.565) (end 126.365 77.915) (width 0.25) (layer "F.Cu") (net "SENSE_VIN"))
 (segment (start 121.92 76.835) (end 122.555 76.835) (width 0.25) (layer "F.Cu") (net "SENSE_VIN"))
 (segment (start 124.51 84.265) (end 124.46 84.315) (width 0.25) (layer "F.Cu") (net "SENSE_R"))
 (segment (start 128.27 84.265) (end 124.51 84.265) (width 0.25) (layer "F.Cu") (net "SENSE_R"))
 (segment (start 122.06 84.315) (end 124.46 84.315) (width 0.25) (layer "F.Cu") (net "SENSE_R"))
 (segment (start 121.92 84.455) (end 122.06 84.315) (width 0.25) (layer "F.Cu") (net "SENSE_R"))
 (segment (start 128.27 85.915) (end 128.27 88.77) (width 0.25) (layer "F.Cu") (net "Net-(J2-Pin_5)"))
 (segment (start 128.27 88.77) (end 128.73 89.23) (width 0.25) (layer "F.Cu") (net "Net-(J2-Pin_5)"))
 (segment (start 131.27 91.77) (end 132.445 90.595) (width 0.25) (layer "F.Cu") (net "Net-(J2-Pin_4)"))
 (segment (start 132.445 90.595) (end 132.445 86.82) (width 0.25) (layer "F.Cu") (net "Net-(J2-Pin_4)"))
 (segment (start 132.445 86.82) (end 133.35 85.915) (width 0.25) (layer "F.Cu") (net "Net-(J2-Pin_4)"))
 (segment (start 131.27 89.23) (end 131.27 86.09) (width 0.25) (layer "F.Cu") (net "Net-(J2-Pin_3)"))
 (segment (start 131.27 86.09) (end 131.445 85.915) (width 0.25) (layer "F.Cu") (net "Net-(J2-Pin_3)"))
 (segment (start 133.81 87.36) (end 135.255 85.915) (width 0.25) (layer "F.Cu") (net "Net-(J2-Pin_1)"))
 (segment (start 133.81 89.23) (end 133.81 87.36) (width 0.25) (layer "F.Cu") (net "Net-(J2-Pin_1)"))
 (segment (start 128.73 91.77) (end 129.905 90.595) (width 0.25) (layer "F.Cu") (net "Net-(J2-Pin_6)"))
 (segment (start 129.905 90.595) (end 129.905 84.375) (width 0.25) (layer "F.Cu") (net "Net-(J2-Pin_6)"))
 (segment (start 129.905 84.375) (end 128.27 82.74) (width 0.25) (layer "F.Cu") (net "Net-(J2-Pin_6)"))
 (segment (start 133.81 91.77) (end 135.255 90.325) (width 0.25) (layer "F.Cu") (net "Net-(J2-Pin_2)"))
 (segment (start 135.255 90.325) (end 135.255 87.82) (width 0.25) (layer "F.Cu") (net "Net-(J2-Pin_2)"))
 (segment (start 135.255 87.82) (end 137.16 85.915) (width 0.25) (layer "F.Cu") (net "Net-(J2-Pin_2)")))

